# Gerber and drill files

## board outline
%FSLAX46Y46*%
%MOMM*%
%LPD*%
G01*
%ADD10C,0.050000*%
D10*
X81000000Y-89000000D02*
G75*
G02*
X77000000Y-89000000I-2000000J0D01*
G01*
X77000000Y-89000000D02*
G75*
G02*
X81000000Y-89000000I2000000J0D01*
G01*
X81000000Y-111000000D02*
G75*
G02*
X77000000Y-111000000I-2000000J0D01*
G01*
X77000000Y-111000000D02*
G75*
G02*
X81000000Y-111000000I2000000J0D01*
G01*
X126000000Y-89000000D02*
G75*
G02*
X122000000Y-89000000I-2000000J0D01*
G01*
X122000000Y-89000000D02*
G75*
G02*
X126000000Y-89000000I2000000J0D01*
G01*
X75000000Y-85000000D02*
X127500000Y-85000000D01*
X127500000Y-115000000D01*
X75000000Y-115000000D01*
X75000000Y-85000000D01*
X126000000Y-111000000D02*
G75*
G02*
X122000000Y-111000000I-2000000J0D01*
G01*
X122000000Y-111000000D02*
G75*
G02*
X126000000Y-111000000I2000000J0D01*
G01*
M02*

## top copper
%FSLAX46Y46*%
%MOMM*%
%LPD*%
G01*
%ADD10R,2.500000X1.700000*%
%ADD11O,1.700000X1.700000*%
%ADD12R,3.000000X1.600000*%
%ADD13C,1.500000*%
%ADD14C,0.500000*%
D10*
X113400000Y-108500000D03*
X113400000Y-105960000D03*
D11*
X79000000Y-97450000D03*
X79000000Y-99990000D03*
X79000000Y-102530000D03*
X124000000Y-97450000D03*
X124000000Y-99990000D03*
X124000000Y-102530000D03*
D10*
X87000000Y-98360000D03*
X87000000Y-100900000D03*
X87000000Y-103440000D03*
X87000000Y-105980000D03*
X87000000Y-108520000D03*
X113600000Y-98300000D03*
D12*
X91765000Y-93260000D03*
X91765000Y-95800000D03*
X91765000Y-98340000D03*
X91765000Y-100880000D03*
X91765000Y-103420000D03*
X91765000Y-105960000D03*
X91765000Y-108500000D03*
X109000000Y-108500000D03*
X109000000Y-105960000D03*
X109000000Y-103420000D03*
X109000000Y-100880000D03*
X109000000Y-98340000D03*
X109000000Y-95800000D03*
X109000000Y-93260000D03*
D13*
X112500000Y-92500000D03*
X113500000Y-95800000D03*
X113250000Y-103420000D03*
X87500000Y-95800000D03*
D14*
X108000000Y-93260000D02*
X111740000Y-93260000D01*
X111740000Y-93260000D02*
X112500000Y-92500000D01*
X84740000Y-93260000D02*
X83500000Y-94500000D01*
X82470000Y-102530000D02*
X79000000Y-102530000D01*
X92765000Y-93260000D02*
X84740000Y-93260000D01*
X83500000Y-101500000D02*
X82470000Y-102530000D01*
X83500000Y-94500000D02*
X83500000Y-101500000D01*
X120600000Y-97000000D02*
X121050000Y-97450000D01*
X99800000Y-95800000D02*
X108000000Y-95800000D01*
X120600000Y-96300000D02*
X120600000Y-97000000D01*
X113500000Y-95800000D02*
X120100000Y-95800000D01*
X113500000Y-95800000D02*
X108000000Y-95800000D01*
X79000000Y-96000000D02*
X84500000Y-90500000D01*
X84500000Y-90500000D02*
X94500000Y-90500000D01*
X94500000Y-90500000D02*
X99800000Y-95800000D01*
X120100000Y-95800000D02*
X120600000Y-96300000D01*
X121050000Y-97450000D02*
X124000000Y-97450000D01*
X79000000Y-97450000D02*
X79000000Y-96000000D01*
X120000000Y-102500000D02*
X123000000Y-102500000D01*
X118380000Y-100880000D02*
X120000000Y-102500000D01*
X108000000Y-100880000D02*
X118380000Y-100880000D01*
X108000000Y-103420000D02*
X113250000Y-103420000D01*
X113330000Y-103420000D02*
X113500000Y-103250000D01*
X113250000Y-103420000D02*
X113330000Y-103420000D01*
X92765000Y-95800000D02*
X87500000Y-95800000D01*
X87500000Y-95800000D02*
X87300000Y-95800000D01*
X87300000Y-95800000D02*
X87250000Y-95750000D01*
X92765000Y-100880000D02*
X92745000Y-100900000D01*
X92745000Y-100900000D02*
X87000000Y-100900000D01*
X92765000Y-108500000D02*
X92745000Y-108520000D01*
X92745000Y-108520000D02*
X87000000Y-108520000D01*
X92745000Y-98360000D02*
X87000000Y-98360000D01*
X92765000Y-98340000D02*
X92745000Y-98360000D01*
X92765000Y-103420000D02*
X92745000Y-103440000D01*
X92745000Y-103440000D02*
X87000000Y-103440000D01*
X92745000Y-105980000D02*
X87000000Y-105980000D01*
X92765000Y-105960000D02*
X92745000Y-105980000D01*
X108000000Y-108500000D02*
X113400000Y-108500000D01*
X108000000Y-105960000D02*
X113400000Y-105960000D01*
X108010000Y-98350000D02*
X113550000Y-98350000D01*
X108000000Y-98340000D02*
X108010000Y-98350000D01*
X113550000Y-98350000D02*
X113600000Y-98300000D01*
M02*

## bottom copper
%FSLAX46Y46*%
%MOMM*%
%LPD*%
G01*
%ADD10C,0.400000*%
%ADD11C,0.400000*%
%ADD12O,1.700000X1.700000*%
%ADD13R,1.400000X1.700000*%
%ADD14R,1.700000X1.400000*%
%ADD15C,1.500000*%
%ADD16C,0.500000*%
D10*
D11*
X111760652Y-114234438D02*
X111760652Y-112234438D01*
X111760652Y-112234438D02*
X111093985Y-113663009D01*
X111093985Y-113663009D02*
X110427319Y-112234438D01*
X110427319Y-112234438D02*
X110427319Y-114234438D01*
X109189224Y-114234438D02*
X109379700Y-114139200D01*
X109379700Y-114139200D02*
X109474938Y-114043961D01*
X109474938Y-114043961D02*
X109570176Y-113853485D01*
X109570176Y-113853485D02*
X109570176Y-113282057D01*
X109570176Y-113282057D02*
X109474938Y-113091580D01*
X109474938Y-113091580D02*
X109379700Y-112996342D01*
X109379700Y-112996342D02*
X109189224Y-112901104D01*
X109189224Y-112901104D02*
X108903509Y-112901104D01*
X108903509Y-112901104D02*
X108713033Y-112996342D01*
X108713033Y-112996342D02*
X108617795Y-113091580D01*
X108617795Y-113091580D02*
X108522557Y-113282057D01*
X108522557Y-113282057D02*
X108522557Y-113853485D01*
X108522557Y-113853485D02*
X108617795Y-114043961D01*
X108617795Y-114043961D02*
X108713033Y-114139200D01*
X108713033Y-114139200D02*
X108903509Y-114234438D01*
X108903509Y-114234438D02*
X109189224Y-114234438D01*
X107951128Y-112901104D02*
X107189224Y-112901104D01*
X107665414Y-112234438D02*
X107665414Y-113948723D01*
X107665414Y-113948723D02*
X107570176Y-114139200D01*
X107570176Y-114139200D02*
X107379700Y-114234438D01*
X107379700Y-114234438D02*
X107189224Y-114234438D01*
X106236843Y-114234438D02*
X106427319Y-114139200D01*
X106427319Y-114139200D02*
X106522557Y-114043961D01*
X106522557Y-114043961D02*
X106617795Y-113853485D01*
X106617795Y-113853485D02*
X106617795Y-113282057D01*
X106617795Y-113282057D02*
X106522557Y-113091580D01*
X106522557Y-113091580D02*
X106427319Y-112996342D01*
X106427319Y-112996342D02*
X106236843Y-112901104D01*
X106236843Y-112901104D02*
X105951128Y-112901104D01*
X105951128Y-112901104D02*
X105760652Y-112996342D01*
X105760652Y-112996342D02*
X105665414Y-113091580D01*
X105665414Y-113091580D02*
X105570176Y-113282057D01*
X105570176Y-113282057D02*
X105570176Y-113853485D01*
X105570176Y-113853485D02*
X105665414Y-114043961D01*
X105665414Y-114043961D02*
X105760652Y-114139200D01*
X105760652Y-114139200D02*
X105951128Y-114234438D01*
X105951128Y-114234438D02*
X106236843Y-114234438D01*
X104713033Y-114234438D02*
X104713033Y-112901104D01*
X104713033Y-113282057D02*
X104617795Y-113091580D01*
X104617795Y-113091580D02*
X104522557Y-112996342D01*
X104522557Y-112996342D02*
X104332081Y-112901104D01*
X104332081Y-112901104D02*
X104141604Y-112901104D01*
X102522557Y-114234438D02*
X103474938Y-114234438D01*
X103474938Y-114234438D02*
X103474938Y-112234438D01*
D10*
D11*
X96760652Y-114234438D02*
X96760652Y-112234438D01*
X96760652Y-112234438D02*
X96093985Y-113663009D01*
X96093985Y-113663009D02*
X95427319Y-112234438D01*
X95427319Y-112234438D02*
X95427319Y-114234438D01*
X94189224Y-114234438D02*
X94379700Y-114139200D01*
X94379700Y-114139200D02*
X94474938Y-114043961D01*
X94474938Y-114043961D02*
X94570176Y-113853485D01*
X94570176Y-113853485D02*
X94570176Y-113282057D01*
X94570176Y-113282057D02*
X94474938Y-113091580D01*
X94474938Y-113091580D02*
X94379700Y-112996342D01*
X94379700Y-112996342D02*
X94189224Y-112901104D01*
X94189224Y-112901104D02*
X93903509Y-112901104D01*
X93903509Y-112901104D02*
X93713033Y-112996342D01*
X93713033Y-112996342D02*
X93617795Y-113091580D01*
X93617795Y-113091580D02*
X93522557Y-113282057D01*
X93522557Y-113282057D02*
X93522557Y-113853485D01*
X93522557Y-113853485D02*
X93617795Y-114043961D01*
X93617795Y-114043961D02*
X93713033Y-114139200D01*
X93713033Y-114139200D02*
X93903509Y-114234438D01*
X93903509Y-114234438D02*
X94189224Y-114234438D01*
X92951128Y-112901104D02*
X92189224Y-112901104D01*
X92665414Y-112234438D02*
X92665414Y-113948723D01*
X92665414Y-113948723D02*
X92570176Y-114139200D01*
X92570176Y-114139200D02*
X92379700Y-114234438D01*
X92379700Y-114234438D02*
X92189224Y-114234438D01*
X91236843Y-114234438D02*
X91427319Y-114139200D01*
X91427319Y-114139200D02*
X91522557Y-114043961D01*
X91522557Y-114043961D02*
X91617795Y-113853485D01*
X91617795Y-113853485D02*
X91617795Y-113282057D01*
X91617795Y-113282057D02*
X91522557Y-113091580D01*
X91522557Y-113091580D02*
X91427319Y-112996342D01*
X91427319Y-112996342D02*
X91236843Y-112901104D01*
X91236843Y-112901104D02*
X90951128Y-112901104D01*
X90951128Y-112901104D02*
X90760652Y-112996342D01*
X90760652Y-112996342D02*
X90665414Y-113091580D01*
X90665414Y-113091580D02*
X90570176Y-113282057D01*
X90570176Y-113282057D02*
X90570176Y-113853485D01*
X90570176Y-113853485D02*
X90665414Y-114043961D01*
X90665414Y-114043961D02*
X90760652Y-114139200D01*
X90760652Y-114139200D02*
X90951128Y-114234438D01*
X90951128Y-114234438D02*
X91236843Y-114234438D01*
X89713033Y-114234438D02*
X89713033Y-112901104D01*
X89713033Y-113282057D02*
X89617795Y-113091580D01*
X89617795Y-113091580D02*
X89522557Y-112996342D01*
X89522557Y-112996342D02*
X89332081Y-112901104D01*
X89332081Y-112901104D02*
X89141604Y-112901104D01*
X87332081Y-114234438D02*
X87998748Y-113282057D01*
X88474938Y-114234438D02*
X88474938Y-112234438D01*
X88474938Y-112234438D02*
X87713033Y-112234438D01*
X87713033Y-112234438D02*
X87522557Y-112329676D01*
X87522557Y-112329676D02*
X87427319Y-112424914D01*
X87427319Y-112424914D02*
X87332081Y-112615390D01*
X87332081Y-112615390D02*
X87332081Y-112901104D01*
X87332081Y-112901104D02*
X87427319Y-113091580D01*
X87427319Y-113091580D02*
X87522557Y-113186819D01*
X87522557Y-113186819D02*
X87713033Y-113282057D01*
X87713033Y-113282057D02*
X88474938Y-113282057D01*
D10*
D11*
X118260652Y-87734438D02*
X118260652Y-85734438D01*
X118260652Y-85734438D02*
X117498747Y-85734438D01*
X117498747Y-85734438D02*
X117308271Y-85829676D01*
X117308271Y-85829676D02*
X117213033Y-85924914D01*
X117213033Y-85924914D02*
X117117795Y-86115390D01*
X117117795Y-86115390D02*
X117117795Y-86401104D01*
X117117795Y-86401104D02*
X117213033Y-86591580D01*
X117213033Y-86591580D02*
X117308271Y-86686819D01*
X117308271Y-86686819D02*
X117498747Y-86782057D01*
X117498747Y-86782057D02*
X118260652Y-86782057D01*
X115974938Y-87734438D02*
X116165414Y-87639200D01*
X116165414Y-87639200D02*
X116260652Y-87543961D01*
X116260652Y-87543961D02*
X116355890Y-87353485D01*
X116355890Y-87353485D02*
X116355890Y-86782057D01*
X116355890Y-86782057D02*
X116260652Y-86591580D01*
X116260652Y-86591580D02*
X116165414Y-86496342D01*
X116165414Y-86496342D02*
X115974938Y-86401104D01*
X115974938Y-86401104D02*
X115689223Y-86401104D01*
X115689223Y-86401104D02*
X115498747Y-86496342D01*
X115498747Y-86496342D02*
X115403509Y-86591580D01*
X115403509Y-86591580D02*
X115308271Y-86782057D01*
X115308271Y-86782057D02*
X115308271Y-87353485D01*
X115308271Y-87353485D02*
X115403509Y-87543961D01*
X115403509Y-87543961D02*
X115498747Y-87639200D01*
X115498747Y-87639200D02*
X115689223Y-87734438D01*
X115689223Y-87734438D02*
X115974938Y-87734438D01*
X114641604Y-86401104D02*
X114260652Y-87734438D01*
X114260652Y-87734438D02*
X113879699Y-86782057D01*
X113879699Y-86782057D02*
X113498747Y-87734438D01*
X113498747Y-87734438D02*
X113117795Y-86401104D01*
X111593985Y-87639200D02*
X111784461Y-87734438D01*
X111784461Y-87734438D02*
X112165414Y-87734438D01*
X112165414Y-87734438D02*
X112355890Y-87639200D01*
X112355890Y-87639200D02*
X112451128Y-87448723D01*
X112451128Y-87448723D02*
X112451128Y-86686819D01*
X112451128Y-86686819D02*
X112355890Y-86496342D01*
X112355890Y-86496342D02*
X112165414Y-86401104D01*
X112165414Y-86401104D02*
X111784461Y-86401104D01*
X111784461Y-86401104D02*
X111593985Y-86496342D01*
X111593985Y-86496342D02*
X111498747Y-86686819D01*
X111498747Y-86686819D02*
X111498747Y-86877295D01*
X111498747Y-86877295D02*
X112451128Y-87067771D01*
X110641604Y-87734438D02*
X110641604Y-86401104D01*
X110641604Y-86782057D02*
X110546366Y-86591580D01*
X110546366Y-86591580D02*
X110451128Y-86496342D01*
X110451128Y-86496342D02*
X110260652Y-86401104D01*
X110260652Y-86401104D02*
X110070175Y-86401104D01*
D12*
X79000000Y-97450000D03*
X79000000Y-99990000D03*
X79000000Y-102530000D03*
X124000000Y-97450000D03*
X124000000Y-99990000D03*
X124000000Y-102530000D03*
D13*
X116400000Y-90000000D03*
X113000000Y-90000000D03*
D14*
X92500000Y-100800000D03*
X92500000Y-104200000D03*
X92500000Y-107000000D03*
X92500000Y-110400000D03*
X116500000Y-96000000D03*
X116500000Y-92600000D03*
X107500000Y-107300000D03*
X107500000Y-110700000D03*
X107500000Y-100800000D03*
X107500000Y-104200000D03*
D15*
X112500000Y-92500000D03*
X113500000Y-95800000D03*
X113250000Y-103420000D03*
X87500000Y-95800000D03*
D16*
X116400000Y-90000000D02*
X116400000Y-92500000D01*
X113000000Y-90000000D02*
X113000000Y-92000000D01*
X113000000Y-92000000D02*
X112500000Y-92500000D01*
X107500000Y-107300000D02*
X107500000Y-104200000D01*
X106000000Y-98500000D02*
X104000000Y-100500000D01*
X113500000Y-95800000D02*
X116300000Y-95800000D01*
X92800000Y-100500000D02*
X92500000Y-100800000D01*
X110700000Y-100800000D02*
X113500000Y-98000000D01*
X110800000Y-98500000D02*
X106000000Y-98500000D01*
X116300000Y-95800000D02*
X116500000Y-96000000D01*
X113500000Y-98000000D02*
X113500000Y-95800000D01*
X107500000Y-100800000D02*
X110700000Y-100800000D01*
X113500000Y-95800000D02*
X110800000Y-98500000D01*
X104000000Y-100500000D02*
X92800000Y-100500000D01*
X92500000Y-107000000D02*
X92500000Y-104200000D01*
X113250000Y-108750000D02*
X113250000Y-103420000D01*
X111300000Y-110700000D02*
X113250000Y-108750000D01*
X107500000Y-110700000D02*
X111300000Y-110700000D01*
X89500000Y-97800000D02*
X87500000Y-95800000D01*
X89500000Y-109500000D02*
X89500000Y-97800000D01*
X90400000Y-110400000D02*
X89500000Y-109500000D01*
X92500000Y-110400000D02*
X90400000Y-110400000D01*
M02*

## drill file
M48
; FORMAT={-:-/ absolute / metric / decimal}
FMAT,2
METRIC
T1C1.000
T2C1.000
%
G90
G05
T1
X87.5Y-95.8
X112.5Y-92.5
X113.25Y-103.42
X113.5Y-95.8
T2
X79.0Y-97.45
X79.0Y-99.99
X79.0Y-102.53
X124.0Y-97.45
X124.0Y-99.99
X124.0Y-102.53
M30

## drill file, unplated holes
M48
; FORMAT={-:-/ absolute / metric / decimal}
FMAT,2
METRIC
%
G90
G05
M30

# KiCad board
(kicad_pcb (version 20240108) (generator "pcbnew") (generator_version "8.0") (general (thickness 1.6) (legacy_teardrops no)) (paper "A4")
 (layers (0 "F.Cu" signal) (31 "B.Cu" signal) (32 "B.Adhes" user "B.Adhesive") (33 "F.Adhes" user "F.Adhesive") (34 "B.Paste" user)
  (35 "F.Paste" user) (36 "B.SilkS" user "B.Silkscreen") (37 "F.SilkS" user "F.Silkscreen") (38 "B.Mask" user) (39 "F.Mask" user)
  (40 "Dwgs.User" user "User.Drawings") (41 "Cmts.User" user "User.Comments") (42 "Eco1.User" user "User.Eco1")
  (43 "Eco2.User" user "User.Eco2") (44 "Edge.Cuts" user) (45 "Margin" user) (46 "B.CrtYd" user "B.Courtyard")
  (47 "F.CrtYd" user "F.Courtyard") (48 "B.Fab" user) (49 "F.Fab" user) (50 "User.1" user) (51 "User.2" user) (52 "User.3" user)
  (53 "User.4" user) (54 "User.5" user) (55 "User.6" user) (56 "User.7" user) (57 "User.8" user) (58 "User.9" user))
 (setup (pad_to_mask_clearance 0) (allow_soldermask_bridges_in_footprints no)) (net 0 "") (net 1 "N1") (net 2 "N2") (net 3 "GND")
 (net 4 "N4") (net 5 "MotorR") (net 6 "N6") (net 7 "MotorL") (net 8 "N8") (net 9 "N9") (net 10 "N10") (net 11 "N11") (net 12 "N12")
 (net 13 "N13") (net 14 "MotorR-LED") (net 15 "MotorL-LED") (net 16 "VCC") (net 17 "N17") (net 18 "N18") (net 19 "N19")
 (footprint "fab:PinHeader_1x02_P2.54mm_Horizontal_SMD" (layer "F.Cu") (at 113.4 108.5 180)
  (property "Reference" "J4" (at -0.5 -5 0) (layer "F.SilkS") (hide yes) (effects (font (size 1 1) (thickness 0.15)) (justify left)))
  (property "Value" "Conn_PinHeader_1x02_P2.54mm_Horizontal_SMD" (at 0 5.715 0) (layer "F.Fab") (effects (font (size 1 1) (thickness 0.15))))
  (pad "1" smd rect (at 0 0 180) (size 2.5 1.7) (layers "F.Cu" "F.Paste" "F.Mask") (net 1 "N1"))
  (pad "2" smd rect (at 0 2.54 180) (size 2.5 1.7) (layers "F.Cu" "F.Paste" "F.Mask") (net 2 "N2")))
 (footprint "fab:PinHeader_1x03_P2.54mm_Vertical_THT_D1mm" (layer "F.Cu") (at 79 97.45)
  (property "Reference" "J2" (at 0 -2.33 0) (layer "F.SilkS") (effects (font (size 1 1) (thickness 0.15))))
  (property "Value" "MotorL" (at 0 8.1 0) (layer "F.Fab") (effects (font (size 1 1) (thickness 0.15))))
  (pad "1" thru_hole oval (at 0 0) (size 1.7 1.7) (drill 1) (layers "*.Cu" "*.Mask") (remove_unused_layers no) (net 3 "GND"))
  (pad "2" thru_hole oval (at 0 2.54) (size 1.7 1.7) (drill 1) (layers "*.Cu" "*.Mask") (remove_unused_layers no) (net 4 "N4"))
  (pad "3" thru_hole oval (at 0 5.08) (size 1.7 1.7) (drill 1) (layers "*.Cu" "*.Mask") (remove_unused_layers no) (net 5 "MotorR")))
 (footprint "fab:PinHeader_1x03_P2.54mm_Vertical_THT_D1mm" (layer "F.Cu") (at 124 97.45)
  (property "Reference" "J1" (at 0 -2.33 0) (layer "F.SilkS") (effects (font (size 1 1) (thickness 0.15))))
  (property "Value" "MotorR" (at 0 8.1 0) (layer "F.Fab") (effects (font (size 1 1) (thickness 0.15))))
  (pad "1" thru_hole oval (at 0 0) (size 1.7 1.7) (drill 1) (layers "*.Cu" "*.Mask") (remove_unused_layers no) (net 3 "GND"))
  (pad "2" thru_hole oval (at 0 2.54) (size 1.7 1.7) (drill 1) (layers "*.Cu" "*.Mask") (remove_unused_layers no) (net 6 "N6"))
  (pad "3" thru_hole oval (at 0 5.08) (size 1.7 1.7) (drill 1) (layers "*.Cu" "*.Mask") (remove_unused_layers no) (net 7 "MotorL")))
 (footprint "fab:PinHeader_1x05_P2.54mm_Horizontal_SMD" (layer "F.Cu") (at 87 98.36)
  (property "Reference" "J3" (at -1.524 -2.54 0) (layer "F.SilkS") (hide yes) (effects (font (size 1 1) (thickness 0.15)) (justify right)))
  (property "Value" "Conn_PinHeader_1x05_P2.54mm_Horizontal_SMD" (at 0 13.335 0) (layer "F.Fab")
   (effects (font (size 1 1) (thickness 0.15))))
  (pad "1" smd rect (at 0 0) (size 2.5 1.7) (layers "F.Cu" "F.Paste" "F.Mask") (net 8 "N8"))
  (pad "2" smd rect (at 0 2.54) (size 2.5 1.7) (layers "F.Cu" "F.Paste" "F.Mask") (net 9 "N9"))
  (pad "3" smd rect (at 0 5.08) (size 2.5 1.7) (layers "F.Cu" "F.Paste" "F.Mask") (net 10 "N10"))
  (pad "4" smd rect (at 0 7.62) (size 2.5 1.7) (layers "F.Cu" "F.Paste" "F.Mask") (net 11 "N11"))
  (pad "5" smd rect (at 0 10.16) (size 2.5 1.7) (layers "F.Cu" "F.Paste" "F.Mask") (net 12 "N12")))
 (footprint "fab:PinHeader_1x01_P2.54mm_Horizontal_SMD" (layer "F.Cu") (at 113.6 98.3)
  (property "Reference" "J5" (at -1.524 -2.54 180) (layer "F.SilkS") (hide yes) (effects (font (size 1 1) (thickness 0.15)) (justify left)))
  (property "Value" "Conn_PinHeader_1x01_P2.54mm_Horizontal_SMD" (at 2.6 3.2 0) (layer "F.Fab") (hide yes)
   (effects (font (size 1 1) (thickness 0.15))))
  (pad "1" smd rect (at 0 0) (size 2.5 1.7) (layers "F.Cu" "F.Paste" "F.Mask") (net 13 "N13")))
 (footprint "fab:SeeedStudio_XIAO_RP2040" (layer "F.Cu") (at 100.38 100.88)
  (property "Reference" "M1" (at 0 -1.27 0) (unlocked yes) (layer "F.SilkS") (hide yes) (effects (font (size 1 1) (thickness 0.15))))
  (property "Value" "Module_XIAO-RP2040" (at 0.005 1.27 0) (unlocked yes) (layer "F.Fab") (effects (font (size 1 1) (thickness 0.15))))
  (pad "1" smd rect (at -7.615 -7.62) (size 3 1.6) (drill (offset -1 0)) (layers "F.Cu" "F.Paste" "F.Mask") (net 5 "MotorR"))
  (pad "2" smd rect (at -7.615 -5.08) (size 3 1.6) (drill (offset -1 0)) (layers "F.Cu" "F.Paste" "F.Mask") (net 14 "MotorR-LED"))
  (pad "3" smd rect (at -7.615 -2.54) (size 3 1.6) (drill (offset -1 0)) (layers "F.Cu" "F.Paste" "F.Mask") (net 8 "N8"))
  (pad "4" smd rect (at -7.615 0) (size 3 1.6) (drill (offset -1 0)) (layers "F.Cu" "F.Paste" "F.Mask") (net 9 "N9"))
  (pad "5" smd rect (at -7.615 2.54) (size 3 1.6) (drill (offset -1 0)) (layers "F.Cu" "F.Paste" "F.Mask") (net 10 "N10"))
  (pad "6" smd rect (at -7.615 5.08) (size 3 1.6) (drill (offset -1 0)) (layers "F.Cu" "F.Paste" "F.Mask") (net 11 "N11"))
  (pad "7" smd rect (at -7.615 7.62) (size 3 1.6) (drill (offset -1 0)) (layers "F.Cu" "F.Paste" "F.Mask") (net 12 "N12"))
  (pad "8" smd rect (at 7.62 7.62) (size 3 1.6) (drill (offset 1 0)) (layers "F.Cu" "F.Paste" "F.Mask") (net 1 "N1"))
  (pad "9" smd rect (at 7.62 5.08) (size 3 1.6) (drill (offset 1 0)) (layers "F.Cu" "F.Paste" "F.Mask") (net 2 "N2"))
  (pad "10" smd rect (at 7.62 2.54) (size 3 1.6) (drill (offset 1 0)) (layers "F.Cu" "F.Paste" "F.Mask") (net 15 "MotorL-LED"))
  (pad "11" smd rect (at 7.62 0) (size 3 1.6) (drill (offset 1 0)) (layers "F.Cu" "F.Paste" "F.Mask") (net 7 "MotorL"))
  (pad "12" smd rect (at 7.62 -2.54) (size 3 1.6) (drill (offset 1 0)) (layers "F.Cu" "F.Paste" "F.Mask") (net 13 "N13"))
  (pad "13" smd rect (at 7.62 -5.08) (size 3 1.6) (drill (offset 1 0)) (layers "F.Cu" "F.Paste" "F.Mask") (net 3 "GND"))
  (pad "14" smd rect (at 7.62 -7.62) (size 3 1.6) (drill (offset 1 0)) (layers "F.Cu" "F.Paste" "F.Mask") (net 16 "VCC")))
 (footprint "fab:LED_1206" (layer "B.Cu") (at 114.7 90 180)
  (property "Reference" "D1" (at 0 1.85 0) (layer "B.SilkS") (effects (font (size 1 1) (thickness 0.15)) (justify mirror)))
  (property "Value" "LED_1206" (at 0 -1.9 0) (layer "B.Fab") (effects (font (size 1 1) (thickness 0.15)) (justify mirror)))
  (pad "1" smd rect (at -1.7 0 180) (size 1.4 1.7) (layers "B.Cu" "B.Paste" "B.Mask") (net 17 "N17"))
  (pad "2" smd rect (at 1.7 0 180) (size 1.4 1.7) (layers "B.Cu" "B.Paste" "B.Mask") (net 16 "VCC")))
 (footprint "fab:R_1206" (layer "B.Cu") (at 92.5 102.5 -90)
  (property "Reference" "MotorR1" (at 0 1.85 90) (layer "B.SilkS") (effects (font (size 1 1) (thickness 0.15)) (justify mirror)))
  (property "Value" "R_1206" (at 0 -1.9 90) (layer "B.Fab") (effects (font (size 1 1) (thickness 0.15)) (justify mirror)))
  (pad "1" smd rect (at -1.7 0 270) (size 1.4 1.7) (layers "B.Cu" "B.Paste" "B.Mask") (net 3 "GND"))
  (pad "2" smd rect (at 1.7 0 270) (size 1.4 1.7) (layers "B.Cu" "B.Paste" "B.Mask") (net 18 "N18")))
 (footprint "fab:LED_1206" (layer "B.Cu") (at 92.5 108.7 -90)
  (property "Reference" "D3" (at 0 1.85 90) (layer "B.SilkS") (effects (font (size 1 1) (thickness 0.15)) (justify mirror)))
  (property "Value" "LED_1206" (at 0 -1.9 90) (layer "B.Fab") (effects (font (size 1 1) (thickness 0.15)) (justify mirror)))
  (pad "1" smd rect (at -1.7 0 270) (size 1.4 1.7) (layers "B.Cu" "B.Paste" "B.Mask") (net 18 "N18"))
  (pad "2" smd rect (at 1.7 0 270) (size 1.4 1.7) (layers "B.Cu" "B.Paste" "B.Mask") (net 14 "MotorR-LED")))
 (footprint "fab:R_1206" (layer "B.Cu") (at 116.5 94.3 90)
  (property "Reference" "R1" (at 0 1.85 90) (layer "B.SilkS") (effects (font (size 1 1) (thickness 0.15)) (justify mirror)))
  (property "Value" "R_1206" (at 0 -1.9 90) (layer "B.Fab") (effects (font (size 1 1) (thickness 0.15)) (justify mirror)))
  (pad "1" smd rect (at -1.7 0 90) (size 1.4 1.7) (layers "B.Cu" "B.Paste" "B.Mask") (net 3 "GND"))
  (pad "2" smd rect (at 1.7 0 90) (size 1.4 1.7) (layers "B.Cu" "B.Paste" "B.Mask") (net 17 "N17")))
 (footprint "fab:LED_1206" (layer "B.Cu") (at 107.5 109 -90)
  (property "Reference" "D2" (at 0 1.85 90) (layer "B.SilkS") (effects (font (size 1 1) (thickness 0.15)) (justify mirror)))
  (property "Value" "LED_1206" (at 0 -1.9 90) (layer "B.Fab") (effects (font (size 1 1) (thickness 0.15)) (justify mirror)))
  (pad "1" smd rect (at -1.7 0 270) (size 1.4 1.7) (layers "B.Cu" "B.Paste" "B.Mask") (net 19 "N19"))
  (pad "2" smd rect (at 1.7 0 270) (size 1.4 1.7) (layers "B.Cu" "B.Paste" "B.Mask") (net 15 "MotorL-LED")))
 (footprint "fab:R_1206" (layer "B.Cu") (at 107.5 102.5 -90)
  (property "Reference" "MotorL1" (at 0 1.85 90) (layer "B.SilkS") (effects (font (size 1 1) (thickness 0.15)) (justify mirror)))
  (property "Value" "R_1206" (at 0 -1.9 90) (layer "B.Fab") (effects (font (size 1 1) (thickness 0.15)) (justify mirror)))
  (pad "1" smd rect (at -1.7 0 270) (size 1.4 1.7) (layers "B.Cu" "B.Paste" "B.Mask") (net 3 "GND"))
  (pad "2" smd rect (at 1.7 0 270) (size 1.4 1.7) (layers "B.Cu" "B.Paste" "B.Mask") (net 19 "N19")))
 (gr_circle (center 79 89) (end 79 87) (stroke (width 0.05) (type default)) (fill none) (layer "Edge.Cuts"))
 (gr_circle (center 79 111) (end 79 109) (stroke (width 0.05) (type default)) (fill none) (layer "Edge.Cuts"))
 (gr_circle (center 124 89) (end 124 87) (stroke (width 0.05) (type default)) (fill none) (layer "Edge.Cuts"))
 (gr_rect (start 75 85) (end 127.5 115) (stroke (width 0.05) (type default)) (fill none) (layer "Edge.Cuts"))
 (gr_circle (center 124 111) (end 126 111) (stroke (width 0.05) (type default)) (fill none) (layer "Edge.Cuts"))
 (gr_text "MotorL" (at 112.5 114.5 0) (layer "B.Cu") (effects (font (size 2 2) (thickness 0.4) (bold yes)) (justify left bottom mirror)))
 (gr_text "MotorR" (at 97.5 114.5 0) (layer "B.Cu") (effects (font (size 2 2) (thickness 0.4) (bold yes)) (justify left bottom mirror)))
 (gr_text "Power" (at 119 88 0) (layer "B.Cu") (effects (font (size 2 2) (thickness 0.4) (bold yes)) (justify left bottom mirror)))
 (segment (start 116.4 90) (end 116.4 92.5) (width 0.5) (layer "B.Cu") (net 17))
 (segment (start 108 93.26) (end 111.74 93.26) (width 0.5) (layer "F.Cu") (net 16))
 (segment (start 111.74 93.26) (end 112.5 92.5) (width 0.5) (layer "F.Cu") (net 16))
 (via (at 112.5 92.5) (size 1.5) (drill 1) (layers "F.Cu" "B.Cu") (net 16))
 (segment (start 113 90) (end 113 92) (width 0.5) (layer "B.Cu") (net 16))
 (segment (start 113 92) (end 112.5 92.5) (width 0.5) (layer "B.Cu") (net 16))
 (segment (start 107.5 107.3) (end 107.5 104.2) (width 0.5) (layer "B.Cu") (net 19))
 (segment (start 84.74 93.26) (end 83.5 94.5) (width 0.5) (layer "F.Cu") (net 5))
 (segment (start 82.47 102.53) (end 79 102.53) (width 0.5) (layer "F.Cu") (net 5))
 (segment (start 92.765 93.26) (end 84.74 93.26) (width 0.5) (layer "F.Cu") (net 5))
 (segment (start 83.5 101.5) (end 82.47 102.53) (width 0.5) (layer "F.Cu") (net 5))
 (segment (start 83.5 94.5) (end 83.5 101.5) (width 0.5) (layer "F.Cu") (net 5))
 (segment (start 120.6 97) (end 121.05 97.45) (width 0.5) (layer "F.Cu") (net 3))
 (segment (start 99.8 95.8) (end 108 95.8) (width 0.5) (layer "F.Cu") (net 3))
 (segment (start 120.6 96.3) (end 120.6 97) (width 0.5) (layer "F.Cu") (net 3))
 (segment (start 113.5 95.8) (end 120.1 95.8) (width 0.5) (layer "F.Cu") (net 3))
 (segment (start 113.5 95.8) (end 108 95.8) (width 0.5) (layer "F.Cu") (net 3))
 (segment (start 79 96) (end 84.5 90.5) (width 0.5) (layer "F.Cu") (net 3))
 (segment (start 84.5 90.5) (end 94.5 90.5) (width 0.5) (layer "F.Cu") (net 3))
 (segment (start 94.5 90.5) (end 99.8 95.8) (width 0.5) (layer "F.Cu") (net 3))
 (segment (start 120.1 95.8) (end 120.6 96.3) (width 0.5) (layer "F.Cu") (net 3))
 (segment (start 121.05 97.45) (end 124 97.45) (width 0.5) (layer "F.Cu") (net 3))
 (segment (start 79 97.45) (end 79 96) (width 0.5) (layer "F.Cu") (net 3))
 (via (at 113.5 95.8) (size 1.5) (drill 1) (layers "F.Cu" "B.Cu") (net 3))
 (segment (start 106 98.5) (end 104 100.5) (width 0.5) (layer "B.Cu") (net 3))
 (segment (start 113.5 95.8) (end 116.3 95.8) (width 0.5) (layer "B.Cu") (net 3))
 (segment (start 92.8 100.5) (end 92.5 100.8) (width 0.5) (layer "B.Cu") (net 3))
 (segment (start 110.7 100.8) (end 113.5 98) (width 0.5) (layer "B.Cu") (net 3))
 (segment (start 110.8 98.5) (end 106 98.5) (width 0.5) (layer "B.Cu") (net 3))
 (segment (start 116.3 95.8) (end 116.5 96) (width 0.5) (layer "B.Cu") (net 3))
 (segment (start 113.5 98) (end 113.5 95.8) (width 0.5) (layer "B.Cu") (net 3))
 (segment (start 107.5 100.8) (end 110.7 100.8) (width 0.5) (layer "B.Cu") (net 3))
 (segment (start 113.5 95.8) (end 110.8 98.5) (width 0.5) (layer "B.Cu") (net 3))
 (segment (start 104 100.5) (end 92.8 100.5) (width 0.5) (layer "B.Cu") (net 3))
 (segment (start 120 102.5) (end 123 102.5) (width 0.5) (layer "F.Cu") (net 7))
 (segment (start 118.38 100.88) (end 120 102.5) (width 0.5) (layer "F.Cu") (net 7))
 (segment (start 108 100.88) (end 118.38 100.88) (width 0.5) (layer "F.Cu") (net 7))
 (segment (start 92.5 107) (end 92.5 104.2) (width 0.5) (layer "B.Cu") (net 18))
 (segment (start 108 103.42) (end 113.25 103.42) (width 0.5) (layer "F.Cu") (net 15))
 (segment (start 113.33 103.42) (end 113.5 103.25) (width 0.5) (layer "F.Cu") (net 15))
 (segment (start 113.25 103.42) (end 113.33 103.42) (width 0.5) (layer "F.Cu") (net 15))
 (via (at 113.25 103.42) (size 1.5) (drill 1) (layers "F.Cu" "B.Cu") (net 15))
 (segment (start 113.25 108.75) (end 113.25 103.42) (width 0.5) (layer "B.Cu") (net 15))
 (segment (start 111.3 110.7) (end 113.25 108.75) (width 0.5) (layer "B.Cu") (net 15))
 (segment (start 107.5 110.7) (end 111.3 110.7) (width 0.5) (layer "B.Cu") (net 15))
 (segment (start 92.765 95.8) (end 87.5 95.8) (width 0.5) (layer "F.Cu") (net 14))
 (segment (start 87.5 95.8) (end 87.3 95.8) (width 0.5) (layer "F.Cu") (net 14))
 (segment (start 87.3 95.8) (end 87.25 95.75) (width 0.5) (layer "F.Cu") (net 14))
 (via (at 87.5 95.8) (size 1.5) (drill 1) (layers "F.Cu" "B.Cu") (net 14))
 (segment (start 89.5 97.8) (end 87.5 95.8) (width 0.5) (layer "B.Cu") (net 14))
 (segment (start 89.5 109.5) (end 89.5 97.8) (width 0.5) (layer "B.Cu") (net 14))
 (segment (start 90.4 110.4) (end 89.5 109.5) (width 0.5) (layer "B.Cu") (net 14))
 (segment (start 92.5 110.4) (end 90.4 110.4) (width 0.5) (layer "B.Cu") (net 14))
 (segment (start 92.765 100.88) (end 92.745 100.9) (width 0.5) (layer "F.Cu") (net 9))
 (segment (start 92.745 100.9) (end 87 100.9) (width 0.5) (layer "F.Cu") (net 9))
 (segment (start 92.765 108.5) (end 92.745 108.52) (width 0.5) (layer "F.Cu") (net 12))
 (segment (start 92.745 108.52) (end 87 108.52) (width 0.5) (layer "F.Cu") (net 12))
 (segment (start 92.745 98.36) (end 87 98.36) (width 0.5) (layer "F.Cu") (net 8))
 (segment (start 92.765 98.34) (end 92.745 98.36) (width 0.5) (layer "F.Cu") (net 8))
 (segment (start 92.765 103.42) (end 92.745 103.44) (width 0.5) (layer "F.Cu") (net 10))
 (segment (start 92.745 103.44) (end 87 103.44) (width 0.5) (layer "F.Cu") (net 10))
 (segment (start 92.745 105.98) (end 87 105.98) (width 0.5) (layer "F.Cu") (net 11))
 (segment (start 92.765 105.96) (end 92.745 105.98) (width 0.5) (layer "F.Cu") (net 11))
 (segment (start 108 108.5) (end 113.4 108.5) (width 0.5) (layer "F.Cu") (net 1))
 (segment (start 108 105.96) (end 113.4 105.96) (width 0.5) (layer "F.Cu") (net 2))
 (segment (start 108.01 98.35) (end 113.55 98.35) (width 0.5) (layer "F.Cu") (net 13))
 (segment (start 108 98.34) (end 108.01 98.35) (width 0.5) (layer "F.Cu") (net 13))
 (segment (start 113.55 98.35) (end 113.6 98.3) (width 0.5) (layer "F.Cu") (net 13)))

